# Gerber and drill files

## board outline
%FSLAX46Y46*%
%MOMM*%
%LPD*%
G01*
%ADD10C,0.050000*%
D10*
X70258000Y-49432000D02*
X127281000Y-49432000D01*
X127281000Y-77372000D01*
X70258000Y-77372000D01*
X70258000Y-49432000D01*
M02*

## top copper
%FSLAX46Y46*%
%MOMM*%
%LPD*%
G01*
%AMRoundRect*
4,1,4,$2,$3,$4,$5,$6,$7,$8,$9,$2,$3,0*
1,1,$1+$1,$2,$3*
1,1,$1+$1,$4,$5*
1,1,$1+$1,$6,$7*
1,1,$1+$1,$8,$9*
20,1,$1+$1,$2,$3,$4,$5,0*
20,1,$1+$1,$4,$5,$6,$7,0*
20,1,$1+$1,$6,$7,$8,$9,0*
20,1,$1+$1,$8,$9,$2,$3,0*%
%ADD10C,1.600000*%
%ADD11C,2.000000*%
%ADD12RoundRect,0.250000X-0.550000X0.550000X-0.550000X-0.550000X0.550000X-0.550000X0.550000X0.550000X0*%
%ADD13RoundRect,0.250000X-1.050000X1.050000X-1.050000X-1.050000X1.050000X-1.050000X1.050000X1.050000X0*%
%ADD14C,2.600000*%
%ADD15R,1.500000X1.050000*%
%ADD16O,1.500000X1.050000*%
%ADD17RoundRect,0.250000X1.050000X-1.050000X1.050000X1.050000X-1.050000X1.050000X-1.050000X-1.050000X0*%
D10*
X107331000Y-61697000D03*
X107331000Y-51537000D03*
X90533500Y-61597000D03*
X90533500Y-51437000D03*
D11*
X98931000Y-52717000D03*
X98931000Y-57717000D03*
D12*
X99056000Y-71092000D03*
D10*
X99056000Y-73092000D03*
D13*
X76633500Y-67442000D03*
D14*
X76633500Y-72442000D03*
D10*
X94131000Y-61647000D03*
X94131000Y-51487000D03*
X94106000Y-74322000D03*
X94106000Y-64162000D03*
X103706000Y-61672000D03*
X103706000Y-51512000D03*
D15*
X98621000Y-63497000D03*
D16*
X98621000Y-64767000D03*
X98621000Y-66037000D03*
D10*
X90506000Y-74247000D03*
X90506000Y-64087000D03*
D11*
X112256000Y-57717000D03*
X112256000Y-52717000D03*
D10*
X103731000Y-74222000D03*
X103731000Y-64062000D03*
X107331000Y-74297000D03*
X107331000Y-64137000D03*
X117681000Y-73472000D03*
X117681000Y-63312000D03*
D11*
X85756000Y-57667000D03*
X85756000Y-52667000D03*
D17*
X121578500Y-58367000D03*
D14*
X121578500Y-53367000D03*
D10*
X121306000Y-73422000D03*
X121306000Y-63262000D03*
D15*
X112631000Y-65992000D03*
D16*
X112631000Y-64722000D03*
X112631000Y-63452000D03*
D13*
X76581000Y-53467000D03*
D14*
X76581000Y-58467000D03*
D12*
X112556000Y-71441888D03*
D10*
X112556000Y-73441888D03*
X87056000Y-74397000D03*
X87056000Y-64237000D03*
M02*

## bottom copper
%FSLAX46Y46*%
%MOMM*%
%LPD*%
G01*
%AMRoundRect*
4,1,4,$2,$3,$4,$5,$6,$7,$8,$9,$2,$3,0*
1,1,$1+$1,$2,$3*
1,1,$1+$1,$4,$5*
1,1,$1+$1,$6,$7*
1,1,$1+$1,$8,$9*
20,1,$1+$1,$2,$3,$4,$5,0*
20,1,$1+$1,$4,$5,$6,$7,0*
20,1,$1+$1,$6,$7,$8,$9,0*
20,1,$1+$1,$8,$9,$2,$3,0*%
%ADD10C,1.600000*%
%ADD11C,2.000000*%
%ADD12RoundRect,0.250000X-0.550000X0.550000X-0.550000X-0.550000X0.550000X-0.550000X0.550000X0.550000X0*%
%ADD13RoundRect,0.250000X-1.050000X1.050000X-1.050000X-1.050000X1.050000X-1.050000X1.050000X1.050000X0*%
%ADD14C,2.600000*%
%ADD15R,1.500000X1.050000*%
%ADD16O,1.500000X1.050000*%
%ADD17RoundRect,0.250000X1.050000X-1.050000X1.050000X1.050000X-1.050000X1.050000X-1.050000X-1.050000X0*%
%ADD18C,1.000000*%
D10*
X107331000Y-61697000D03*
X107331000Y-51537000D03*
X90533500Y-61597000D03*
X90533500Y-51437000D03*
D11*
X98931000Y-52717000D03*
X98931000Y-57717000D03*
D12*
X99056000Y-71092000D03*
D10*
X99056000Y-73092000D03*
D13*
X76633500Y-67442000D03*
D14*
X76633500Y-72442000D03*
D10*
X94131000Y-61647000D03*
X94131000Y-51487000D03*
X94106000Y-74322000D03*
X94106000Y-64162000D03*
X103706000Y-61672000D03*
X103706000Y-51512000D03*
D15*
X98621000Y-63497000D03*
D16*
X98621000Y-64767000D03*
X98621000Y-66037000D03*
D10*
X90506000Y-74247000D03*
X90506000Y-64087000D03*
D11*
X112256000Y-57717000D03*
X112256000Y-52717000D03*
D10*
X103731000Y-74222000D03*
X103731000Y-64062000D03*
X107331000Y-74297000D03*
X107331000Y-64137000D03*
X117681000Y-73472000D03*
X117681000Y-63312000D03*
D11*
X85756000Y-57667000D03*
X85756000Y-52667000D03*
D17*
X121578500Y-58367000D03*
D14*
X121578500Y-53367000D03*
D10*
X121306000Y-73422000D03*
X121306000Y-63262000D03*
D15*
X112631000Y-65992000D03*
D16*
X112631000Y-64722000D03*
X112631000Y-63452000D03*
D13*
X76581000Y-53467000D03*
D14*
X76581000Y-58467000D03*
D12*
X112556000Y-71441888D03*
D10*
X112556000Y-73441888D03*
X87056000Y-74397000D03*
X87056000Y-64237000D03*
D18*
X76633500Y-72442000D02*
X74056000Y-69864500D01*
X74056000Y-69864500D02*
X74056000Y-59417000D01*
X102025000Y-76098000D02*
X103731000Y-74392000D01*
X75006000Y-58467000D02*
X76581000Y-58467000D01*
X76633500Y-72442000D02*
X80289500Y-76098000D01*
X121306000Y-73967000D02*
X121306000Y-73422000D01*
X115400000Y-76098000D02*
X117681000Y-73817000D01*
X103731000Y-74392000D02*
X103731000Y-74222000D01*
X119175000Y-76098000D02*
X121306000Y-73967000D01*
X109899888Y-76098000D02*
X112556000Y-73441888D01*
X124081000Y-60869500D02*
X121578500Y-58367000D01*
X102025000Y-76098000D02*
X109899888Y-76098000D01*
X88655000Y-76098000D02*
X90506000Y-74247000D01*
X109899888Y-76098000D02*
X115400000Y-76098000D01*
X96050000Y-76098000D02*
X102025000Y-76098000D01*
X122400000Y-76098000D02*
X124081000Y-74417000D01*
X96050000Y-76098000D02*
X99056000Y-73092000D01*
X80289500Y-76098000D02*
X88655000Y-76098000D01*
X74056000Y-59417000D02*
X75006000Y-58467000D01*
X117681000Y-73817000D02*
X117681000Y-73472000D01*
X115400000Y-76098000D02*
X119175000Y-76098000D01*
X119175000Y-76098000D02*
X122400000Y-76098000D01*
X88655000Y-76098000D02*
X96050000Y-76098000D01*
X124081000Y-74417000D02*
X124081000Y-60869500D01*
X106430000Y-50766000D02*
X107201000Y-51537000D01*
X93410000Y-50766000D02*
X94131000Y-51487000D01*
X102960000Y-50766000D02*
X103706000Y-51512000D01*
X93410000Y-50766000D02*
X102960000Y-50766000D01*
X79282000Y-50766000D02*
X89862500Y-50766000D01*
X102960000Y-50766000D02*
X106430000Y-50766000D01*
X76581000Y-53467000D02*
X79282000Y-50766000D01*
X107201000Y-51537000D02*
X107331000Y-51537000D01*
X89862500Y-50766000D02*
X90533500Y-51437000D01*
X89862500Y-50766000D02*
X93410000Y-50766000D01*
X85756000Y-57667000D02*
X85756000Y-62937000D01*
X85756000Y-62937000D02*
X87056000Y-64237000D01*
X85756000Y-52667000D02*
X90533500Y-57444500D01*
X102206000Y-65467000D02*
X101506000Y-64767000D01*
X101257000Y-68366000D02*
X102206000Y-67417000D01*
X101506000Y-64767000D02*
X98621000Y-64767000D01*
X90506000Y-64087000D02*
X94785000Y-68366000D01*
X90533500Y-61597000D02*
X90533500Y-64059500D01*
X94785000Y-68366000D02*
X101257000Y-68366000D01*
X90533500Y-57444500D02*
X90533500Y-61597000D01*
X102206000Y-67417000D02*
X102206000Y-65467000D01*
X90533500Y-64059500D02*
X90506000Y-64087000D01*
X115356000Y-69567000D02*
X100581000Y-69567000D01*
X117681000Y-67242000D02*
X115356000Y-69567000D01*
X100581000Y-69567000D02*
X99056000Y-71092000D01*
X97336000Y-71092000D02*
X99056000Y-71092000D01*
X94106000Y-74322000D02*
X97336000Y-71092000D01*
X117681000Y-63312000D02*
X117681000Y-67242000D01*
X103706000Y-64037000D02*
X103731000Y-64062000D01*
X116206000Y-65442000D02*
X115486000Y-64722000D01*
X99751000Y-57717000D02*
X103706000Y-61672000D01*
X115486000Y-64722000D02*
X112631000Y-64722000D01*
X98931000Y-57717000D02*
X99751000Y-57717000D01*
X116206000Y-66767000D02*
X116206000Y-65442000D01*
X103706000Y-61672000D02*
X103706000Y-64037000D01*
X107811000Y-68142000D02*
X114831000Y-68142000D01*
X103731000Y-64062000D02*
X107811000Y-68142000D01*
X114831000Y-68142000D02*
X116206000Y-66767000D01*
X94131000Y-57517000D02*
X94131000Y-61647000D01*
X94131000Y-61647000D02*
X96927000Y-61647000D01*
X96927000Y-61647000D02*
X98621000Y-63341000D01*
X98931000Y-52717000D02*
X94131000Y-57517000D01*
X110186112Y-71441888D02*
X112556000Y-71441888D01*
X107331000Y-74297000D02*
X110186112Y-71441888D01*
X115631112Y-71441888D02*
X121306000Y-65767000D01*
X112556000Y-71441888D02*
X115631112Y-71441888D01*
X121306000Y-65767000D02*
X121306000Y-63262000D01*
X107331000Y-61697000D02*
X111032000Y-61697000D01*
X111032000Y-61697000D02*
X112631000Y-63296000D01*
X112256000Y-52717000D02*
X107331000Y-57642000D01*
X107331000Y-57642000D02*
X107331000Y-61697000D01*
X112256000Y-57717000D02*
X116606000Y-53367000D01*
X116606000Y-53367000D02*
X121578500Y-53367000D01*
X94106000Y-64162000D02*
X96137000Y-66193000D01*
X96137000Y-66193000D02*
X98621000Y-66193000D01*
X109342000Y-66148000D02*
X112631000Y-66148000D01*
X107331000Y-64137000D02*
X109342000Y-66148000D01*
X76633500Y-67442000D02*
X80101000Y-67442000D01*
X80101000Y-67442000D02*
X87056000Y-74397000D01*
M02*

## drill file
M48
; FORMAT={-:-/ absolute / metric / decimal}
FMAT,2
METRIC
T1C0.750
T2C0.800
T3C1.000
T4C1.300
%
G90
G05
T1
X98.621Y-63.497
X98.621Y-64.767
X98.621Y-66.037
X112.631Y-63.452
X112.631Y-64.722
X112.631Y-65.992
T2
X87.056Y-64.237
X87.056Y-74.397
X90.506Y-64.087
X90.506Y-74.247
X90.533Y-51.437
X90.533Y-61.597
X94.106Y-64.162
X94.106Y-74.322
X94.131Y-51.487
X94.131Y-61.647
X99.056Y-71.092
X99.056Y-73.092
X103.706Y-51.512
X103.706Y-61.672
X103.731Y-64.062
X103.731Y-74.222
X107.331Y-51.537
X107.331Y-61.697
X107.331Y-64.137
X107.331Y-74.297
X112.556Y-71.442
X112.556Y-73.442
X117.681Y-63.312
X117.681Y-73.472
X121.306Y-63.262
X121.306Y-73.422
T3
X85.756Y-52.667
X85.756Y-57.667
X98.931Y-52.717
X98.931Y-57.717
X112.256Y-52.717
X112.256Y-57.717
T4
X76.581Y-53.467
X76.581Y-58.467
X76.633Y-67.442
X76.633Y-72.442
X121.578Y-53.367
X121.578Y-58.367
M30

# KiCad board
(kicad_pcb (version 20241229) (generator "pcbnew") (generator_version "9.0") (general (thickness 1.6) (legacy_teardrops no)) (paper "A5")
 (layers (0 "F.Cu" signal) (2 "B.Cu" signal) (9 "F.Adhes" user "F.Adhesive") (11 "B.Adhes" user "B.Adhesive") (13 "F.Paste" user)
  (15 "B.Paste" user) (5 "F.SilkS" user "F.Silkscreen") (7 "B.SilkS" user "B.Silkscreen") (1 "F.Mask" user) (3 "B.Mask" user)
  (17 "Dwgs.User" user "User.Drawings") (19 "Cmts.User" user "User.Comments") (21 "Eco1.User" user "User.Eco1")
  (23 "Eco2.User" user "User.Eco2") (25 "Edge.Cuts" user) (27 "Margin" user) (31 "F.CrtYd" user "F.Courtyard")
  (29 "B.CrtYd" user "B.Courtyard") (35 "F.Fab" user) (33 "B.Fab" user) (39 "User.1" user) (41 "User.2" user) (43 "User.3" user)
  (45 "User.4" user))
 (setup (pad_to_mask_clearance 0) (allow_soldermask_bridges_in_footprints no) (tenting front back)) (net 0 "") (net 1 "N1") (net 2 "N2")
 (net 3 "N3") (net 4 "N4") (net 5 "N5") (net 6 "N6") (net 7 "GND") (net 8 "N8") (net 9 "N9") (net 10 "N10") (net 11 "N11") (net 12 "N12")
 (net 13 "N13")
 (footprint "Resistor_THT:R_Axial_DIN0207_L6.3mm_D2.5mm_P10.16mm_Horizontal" (layer "F.Cu") (at 107.331 61.697 90)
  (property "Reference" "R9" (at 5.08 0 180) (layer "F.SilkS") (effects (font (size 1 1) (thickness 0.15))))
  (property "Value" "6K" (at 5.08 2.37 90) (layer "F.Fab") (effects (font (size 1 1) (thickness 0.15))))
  (pad "1" thru_hole circle (at 0 0 90) (size 1.6 1.6) (drill 0.8) (layers "*.Cu" "*.Mask") (remove_unused_layers no) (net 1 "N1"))
  (pad "2" thru_hole circle (at 10.16 0 90) (size 1.6 1.6) (drill 0.8) (layers "*.Cu" "*.Mask") (remove_unused_layers no) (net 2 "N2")))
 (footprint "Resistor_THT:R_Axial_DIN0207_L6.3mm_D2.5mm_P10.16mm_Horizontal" (layer "F.Cu") (at 90.5335 61.597 90)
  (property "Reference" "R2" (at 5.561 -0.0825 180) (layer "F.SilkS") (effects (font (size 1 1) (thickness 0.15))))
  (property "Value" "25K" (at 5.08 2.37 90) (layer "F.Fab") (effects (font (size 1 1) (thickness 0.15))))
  (pad "1" thru_hole circle (at 0 0 90) (size 1.6 1.6) (drill 0.8) (layers "*.Cu" "*.Mask") (remove_unused_layers no) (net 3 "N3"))
  (pad "2" thru_hole circle (at 10.16 0 90) (size 1.6 1.6) (drill 0.8) (layers "*.Cu" "*.Mask") (remove_unused_layers no) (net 2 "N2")))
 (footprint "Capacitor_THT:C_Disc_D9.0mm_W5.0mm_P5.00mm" (layer "F.Cu") (at 98.931 52.717 -90)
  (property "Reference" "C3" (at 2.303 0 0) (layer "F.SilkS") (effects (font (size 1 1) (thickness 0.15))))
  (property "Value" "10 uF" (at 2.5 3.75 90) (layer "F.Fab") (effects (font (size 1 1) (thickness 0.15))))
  (pad "1" thru_hole circle (at 0 0 270) (size 2 2) (drill 1) (layers "*.Cu" "*.Mask") (remove_unused_layers no) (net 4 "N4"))
  (pad "2" thru_hole circle (at 5 0 270) (size 2 2) (drill 1) (layers "*.Cu" "*.Mask") (remove_unused_layers no) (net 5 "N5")))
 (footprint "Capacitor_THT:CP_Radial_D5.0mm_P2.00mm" (layer "F.Cu") (at 99.056 71.092 -90)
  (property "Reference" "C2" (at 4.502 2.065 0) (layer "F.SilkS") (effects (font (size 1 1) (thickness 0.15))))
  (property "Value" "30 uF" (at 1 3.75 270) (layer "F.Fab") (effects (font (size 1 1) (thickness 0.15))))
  (pad "1" thru_hole roundrect (at 0 0 270) (size 1.6 1.6) (drill 0.8) (layers "*.Cu" "*.Mask") (remove_unused_layers no)
   (roundrect_rratio 0.15625) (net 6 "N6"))
  (pad "2" thru_hole circle (at 2 0 270) (size 1.6 1.6) (drill 0.8) (layers "*.Cu" "*.Mask") (remove_unused_layers no) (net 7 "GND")))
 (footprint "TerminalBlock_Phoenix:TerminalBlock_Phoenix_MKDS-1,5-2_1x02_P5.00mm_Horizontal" (layer "F.Cu") (at 76.6335 67.442 -90)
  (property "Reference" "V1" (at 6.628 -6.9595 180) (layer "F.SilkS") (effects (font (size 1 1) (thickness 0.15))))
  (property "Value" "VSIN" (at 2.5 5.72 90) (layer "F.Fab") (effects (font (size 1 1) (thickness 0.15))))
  (pad "1" thru_hole roundrect (at 0 0 270) (size 2.6 2.6) (drill 1.3) (layers "*.Cu" "*.Mask") (remove_unused_layers no)
   (roundrect_rratio 0.096154) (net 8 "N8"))
  (pad "2" thru_hole circle (at 5 0 270) (size 2.6 2.6) (drill 1.3) (layers "*.Cu" "*.Mask") (remove_unused_layers no) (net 7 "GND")))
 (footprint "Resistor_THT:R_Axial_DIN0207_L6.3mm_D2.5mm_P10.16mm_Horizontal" (layer "F.Cu") (at 94.131 61.647 90)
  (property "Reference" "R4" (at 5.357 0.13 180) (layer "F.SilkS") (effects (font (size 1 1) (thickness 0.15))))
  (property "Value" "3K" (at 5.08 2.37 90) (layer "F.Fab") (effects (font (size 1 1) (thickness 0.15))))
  (pad "1" thru_hole circle (at 0 0 90) (size 1.6 1.6) (drill 0.8) (layers "*.Cu" "*.Mask") (remove_unused_layers no) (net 4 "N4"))
  (pad "2" thru_hole circle (at 10.16 0 90) (size 1.6 1.6) (drill 0.8) (layers "*.Cu" "*.Mask") (remove_unused_layers no) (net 2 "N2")))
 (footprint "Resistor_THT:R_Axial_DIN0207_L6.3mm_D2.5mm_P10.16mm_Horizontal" (layer "F.Cu") (at 94.106 74.322 90)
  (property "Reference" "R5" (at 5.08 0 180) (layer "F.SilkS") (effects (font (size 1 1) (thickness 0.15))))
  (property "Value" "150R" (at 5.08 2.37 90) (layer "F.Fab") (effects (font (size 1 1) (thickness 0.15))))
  (pad "1" thru_hole circle (at 0 0 90) (size 1.6 1.6) (drill 0.8) (layers "*.Cu" "*.Mask") (remove_unused_layers no) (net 6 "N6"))
  (pad "2" thru_hole circle (at 10.16 0 90) (size 1.6 1.6) (drill 0.8) (layers "*.Cu" "*.Mask") (remove_unused_layers no) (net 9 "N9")))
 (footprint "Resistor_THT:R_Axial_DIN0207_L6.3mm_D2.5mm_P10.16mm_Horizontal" (layer "F.Cu") (at 103.706 61.672 90)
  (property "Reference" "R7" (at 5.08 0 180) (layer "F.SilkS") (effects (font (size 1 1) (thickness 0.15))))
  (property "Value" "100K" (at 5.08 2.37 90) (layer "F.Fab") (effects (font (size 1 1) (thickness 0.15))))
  (pad "1" thru_hole circle (at 0 0 90) (size 1.6 1.6) (drill 0.8) (layers "*.Cu" "*.Mask") (remove_unused_layers no) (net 5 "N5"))
  (pad "2" thru_hole circle (at 10.16 0 90) (size 1.6 1.6) (drill 0.8) (layers "*.Cu" "*.Mask") (remove_unused_layers no) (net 2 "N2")))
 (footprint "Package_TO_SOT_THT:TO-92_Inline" (layer "F.Cu") (at 98.621 63.497 -90)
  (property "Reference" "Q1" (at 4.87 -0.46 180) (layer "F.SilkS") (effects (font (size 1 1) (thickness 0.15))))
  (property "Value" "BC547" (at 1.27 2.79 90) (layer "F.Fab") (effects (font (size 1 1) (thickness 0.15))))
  (pad "1" thru_hole rect (at 0 0 270) (size 1.05 1.5) (drill 0.75) (layers "*.Cu" "*.Mask") (remove_unused_layers no) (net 4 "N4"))
  (pad "2" thru_hole oval (at 1.27 0 270) (size 1.05 1.5) (drill 0.75) (layers "*.Cu" "*.Mask") (remove_unused_layers no) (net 3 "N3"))
  (pad "3" thru_hole oval (at 2.54 0 270) (size 1.05 1.5) (drill 0.75) (layers "*.Cu" "*.Mask") (remove_unused_layers no) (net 9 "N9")))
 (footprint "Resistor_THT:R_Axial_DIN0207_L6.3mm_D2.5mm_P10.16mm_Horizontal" (layer "F.Cu") (at 90.506 74.247 90)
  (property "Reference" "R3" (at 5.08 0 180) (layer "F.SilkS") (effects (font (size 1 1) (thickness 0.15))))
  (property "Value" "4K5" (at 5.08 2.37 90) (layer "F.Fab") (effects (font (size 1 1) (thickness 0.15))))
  (pad "1" thru_hole circle (at 0 0 90) (size 1.6 1.6) (drill 0.8) (layers "*.Cu" "*.Mask") (remove_unused_layers no) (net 7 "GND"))
  (pad "2" thru_hole circle (at 10.16 0 90) (size 1.6 1.6) (drill 0.8) (layers "*.Cu" "*.Mask") (remove_unused_layers no) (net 3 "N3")))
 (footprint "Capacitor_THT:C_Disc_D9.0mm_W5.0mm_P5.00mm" (layer "F.Cu") (at 112.256 57.717 90)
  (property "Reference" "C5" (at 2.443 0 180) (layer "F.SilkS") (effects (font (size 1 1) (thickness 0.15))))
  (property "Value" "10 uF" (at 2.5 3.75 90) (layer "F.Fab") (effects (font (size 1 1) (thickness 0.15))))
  (pad "1" thru_hole circle (at 0 0 90) (size 2 2) (drill 1) (layers "*.Cu" "*.Mask") (remove_unused_layers no) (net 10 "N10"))
  (pad "2" thru_hole circle (at 5 0 90) (size 2 2) (drill 1) (layers "*.Cu" "*.Mask") (remove_unused_layers no) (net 1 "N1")))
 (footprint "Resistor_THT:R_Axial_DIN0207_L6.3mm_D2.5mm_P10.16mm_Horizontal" (layer "F.Cu") (at 103.731 74.222 90)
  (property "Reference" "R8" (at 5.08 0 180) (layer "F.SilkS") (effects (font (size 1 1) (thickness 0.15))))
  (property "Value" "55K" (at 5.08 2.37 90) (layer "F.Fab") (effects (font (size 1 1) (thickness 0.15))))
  (pad "1" thru_hole circle (at 0 0 90) (size 1.6 1.6) (drill 0.8) (layers "*.Cu" "*.Mask") (remove_unused_layers no) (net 7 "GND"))
  (pad "2" thru_hole circle (at 10.16 0 90) (size 1.6 1.6) (drill 0.8) (layers "*.Cu" "*.Mask") (remove_unused_layers no) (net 5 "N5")))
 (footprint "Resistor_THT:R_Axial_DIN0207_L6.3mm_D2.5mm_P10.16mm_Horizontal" (layer "F.Cu") (at 107.331 74.297 90)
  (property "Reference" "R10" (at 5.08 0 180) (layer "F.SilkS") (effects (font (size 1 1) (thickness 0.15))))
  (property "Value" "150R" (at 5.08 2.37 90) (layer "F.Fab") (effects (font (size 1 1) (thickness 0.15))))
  (pad "1" thru_hole circle (at 0 0 90) (size 1.6 1.6) (drill 0.8) (layers "*.Cu" "*.Mask") (remove_unused_layers no) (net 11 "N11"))
  (pad "2" thru_hole circle (at 10.16 0 90) (size 1.6 1.6) (drill 0.8) (layers "*.Cu" "*.Mask") (remove_unused_layers no) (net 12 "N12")))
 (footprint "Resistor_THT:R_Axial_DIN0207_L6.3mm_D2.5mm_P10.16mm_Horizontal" (layer "F.Cu") (at 117.681 73.472 90)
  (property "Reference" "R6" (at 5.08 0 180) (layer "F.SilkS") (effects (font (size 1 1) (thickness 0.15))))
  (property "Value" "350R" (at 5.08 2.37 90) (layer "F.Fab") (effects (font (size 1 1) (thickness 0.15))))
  (pad "1" thru_hole circle (at 0 0 90) (size 1.6 1.6) (drill 0.8) (layers "*.Cu" "*.Mask") (remove_unused_layers no) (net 7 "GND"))
  (pad "2" thru_hole circle (at 10.16 0 90) (size 1.6 1.6) (drill 0.8) (layers "*.Cu" "*.Mask") (remove_unused_layers no) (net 6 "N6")))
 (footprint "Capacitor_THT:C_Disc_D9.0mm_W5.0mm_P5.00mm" (layer "F.Cu") (at 85.756 57.667 90)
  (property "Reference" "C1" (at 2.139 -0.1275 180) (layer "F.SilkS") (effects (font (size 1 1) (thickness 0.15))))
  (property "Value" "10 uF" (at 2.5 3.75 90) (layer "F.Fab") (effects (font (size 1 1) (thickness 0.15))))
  (pad "1" thru_hole circle (at 0 0 90) (size 2 2) (drill 1) (layers "*.Cu" "*.Mask") (remove_unused_layers no) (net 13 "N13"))
  (pad "2" thru_hole circle (at 5 0 90) (size 2 2) (drill 1) (layers "*.Cu" "*.Mask") (remove_unused_layers no) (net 3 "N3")))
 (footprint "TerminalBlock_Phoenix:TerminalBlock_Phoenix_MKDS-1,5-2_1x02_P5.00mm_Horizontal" (layer "F.Cu") (at 121.5785 58.367 90)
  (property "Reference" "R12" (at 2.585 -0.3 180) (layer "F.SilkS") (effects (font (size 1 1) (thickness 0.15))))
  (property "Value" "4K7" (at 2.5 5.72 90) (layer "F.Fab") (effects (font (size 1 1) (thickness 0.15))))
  (pad "1" thru_hole roundrect (at 0 0 90) (size 2.6 2.6) (drill 1.3) (layers "*.Cu" "*.Mask") (remove_unused_layers no)
   (roundrect_rratio 0.096154) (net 7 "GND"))
  (pad "2" thru_hole circle (at 5 0 90) (size 2.6 2.6) (drill 1.3) (layers "*.Cu" "*.Mask") (remove_unused_layers no) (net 10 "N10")))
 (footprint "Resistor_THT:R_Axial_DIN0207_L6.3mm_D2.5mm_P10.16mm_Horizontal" (layer "F.Cu") (at 121.306 73.422 90)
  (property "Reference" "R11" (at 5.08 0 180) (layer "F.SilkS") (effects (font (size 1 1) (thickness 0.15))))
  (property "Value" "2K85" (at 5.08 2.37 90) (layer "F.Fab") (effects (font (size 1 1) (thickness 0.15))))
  (pad "1" thru_hole circle (at 0 0 90) (size 1.6 1.6) (drill 0.8) (layers "*.Cu" "*.Mask") (remove_unused_layers no) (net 7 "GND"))
  (pad "2" thru_hole circle (at 10.16 0 90) (size 1.6 1.6) (drill 0.8) (layers "*.Cu" "*.Mask") (remove_unused_layers no) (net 11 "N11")))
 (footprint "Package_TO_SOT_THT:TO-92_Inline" (layer "F.Cu") (at 112.631 65.992 90)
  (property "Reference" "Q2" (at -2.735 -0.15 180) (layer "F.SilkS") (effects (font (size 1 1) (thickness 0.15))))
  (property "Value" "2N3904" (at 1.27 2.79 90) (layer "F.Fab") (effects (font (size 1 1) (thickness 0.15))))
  (pad "1" thru_hole rect (at 0 0 90) (size 1.05 1.5) (drill 0.75) (layers "*.Cu" "*.Mask") (remove_unused_layers no) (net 12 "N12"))
  (pad "2" thru_hole oval (at 1.27 0 90) (size 1.05 1.5) (drill 0.75) (layers "*.Cu" "*.Mask") (remove_unused_layers no) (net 5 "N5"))
  (pad "3" thru_hole oval (at 2.54 0 90) (size 1.05 1.5) (drill 0.75) (layers "*.Cu" "*.Mask") (remove_unused_layers no) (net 1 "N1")))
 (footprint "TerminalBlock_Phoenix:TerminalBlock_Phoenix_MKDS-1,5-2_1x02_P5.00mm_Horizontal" (layer "F.Cu") (at 76.581 53.467 -90)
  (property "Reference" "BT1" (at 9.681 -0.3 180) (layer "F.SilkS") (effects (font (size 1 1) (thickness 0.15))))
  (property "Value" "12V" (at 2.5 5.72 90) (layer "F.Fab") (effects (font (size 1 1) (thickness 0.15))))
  (pad "1" thru_hole roundrect (at 0 0 270) (size 2.6 2.6) (drill 1.3) (layers "*.Cu" "*.Mask") (remove_unused_layers no)
   (roundrect_rratio 0.096154) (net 2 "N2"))
  (pad "2" thru_hole circle (at 5 0 270) (size 2.6 2.6) (drill 1.3) (layers "*.Cu" "*.Mask") (remove_unused_layers no) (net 7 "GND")))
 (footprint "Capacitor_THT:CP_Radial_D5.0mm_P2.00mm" (layer "F.Cu") (at 112.556 71.441888 -90)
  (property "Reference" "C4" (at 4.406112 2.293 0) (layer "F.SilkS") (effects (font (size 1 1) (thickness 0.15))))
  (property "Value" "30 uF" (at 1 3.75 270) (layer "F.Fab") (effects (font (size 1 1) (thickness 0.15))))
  (pad "1" thru_hole roundrect (at 0 0 270) (size 1.6 1.6) (drill 0.8) (layers "*.Cu" "*.Mask") (remove_unused_layers no)
   (roundrect_rratio 0.15625) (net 11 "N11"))
  (pad "2" thru_hole circle (at 2 0 270) (size 1.6 1.6) (drill 0.8) (layers "*.Cu" "*.Mask") (remove_unused_layers no) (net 7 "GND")))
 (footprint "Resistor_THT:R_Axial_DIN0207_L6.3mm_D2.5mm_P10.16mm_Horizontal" (layer "F.Cu") (at 87.056 74.397 90)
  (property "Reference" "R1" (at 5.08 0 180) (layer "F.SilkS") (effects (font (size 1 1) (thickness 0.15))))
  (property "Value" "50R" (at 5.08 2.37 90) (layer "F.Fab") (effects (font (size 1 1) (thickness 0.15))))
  (pad "1" thru_hole circle (at 0 0 90) (size 1.6 1.6) (drill 0.8) (layers "*.Cu" "*.Mask") (remove_unused_layers no) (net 8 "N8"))
  (pad "2" thru_hole circle (at 10.16 0 90) (size 1.6 1.6) (drill 0.8) (layers "*.Cu" "*.Mask") (remove_unused_layers no) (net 13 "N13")))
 (gr_rect (start 70.258 49.432) (end 127.281 77.372) (stroke (width 0.05) (type default)) (fill no) (layer "Edge.Cuts"))
 (segment (start 76.6335 72.442) (end 74.056 69.8645) (width 1) (layer "B.Cu") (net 7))
 (segment (start 74.056 69.8645) (end 74.056 59.417) (width 1) (layer "B.Cu") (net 7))
 (segment (start 102.025 76.098) (end 103.731 74.392) (width 1) (layer "B.Cu") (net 7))
 (segment (start 75.006 58.467) (end 76.581 58.467) (width 1) (layer "B.Cu") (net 7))
 (segment (start 76.6335 72.442) (end 80.2895 76.098) (width 1) (layer "B.Cu") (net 7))
 (segment (start 121.306 73.967) (end 121.306 73.422) (width 1) (layer "B.Cu") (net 7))
 (segment (start 115.4 76.098) (end 117.681 73.817) (width 1) (layer "B.Cu") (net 7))
 (segment (start 103.731 74.392) (end 103.731 74.222) (width 1) (layer "B.Cu") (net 7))
 (segment (start 119.175 76.098) (end 121.306 73.967) (width 1) (layer "B.Cu") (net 7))
 (segment (start 109.899888 76.098) (end 112.556 73.441888) (width 1) (layer "B.Cu") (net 7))
 (segment (start 124.081 60.8695) (end 121.5785 58.367) (width 1) (layer "B.Cu") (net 7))
 (segment (start 102.025 76.098) (end 109.899888 76.098) (width 1) (layer "B.Cu") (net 7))
 (segment (start 88.655 76.098) (end 90.506 74.247) (width 1) (layer "B.Cu") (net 7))
 (segment (start 109.899888 76.098) (end 115.4 76.098) (width 1) (layer "B.Cu") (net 7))
 (segment (start 96.05 76.098) (end 102.025 76.098) (width 1) (layer "B.Cu") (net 7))
 (segment (start 122.4 76.098) (end 124.081 74.417) (width 1) (layer "B.Cu") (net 7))
 (segment (start 96.05 76.098) (end 99.056 73.092) (width 1) (layer "B.Cu") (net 7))
 (segment (start 80.2895 76.098) (end 88.655 76.098) (width 1) (layer "B.Cu") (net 7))
 (segment (start 74.056 59.417) (end 75.006 58.467) (width 1) (layer "B.Cu") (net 7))
 (segment (start 117.681 73.817) (end 117.681 73.472) (width 1) (layer "B.Cu") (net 7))
 (segment (start 115.4 76.098) (end 119.175 76.098) (width 1) (layer "B.Cu") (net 7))
 (segment (start 119.175 76.098) (end 122.4 76.098) (width 1) (layer "B.Cu") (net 7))
 (segment (start 88.655 76.098) (end 96.05 76.098) (width 1) (layer "B.Cu") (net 7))
 (segment (start 124.081 74.417) (end 124.081 60.8695) (width 1) (layer "B.Cu") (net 7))
 (segment (start 106.43 50.766) (end 107.201 51.537) (width 1) (layer "B.Cu") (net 2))
 (segment (start 93.41 50.766) (end 94.131 51.487) (width 1) (layer "B.Cu") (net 2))
 (segment (start 102.96 50.766) (end 103.706 51.512) (width 1) (layer "B.Cu") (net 2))
 (segment (start 93.41 50.766) (end 102.96 50.766) (width 1) (layer "B.Cu") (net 2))
 (segment (start 79.282 50.766) (end 89.8625 50.766) (width 1) (layer "B.Cu") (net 2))
 (segment (start 102.96 50.766) (end 106.43 50.766) (width 1) (layer "B.Cu") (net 2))
 (segment (start 76.581 53.467) (end 79.282 50.766) (width 1) (layer "B.Cu") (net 2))
 (segment (start 107.201 51.537) (end 107.331 51.537) (width 1) (layer "B.Cu") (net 2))
 (segment (start 89.8625 50.766) (end 90.5335 51.437) (width 1) (layer "B.Cu") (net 2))
 (segment (start 89.8625 50.766) (end 93.41 50.766) (width 1) (layer "B.Cu") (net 2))
 (segment (start 85.756 57.667) (end 85.756 62.937) (width 1) (layer "B.Cu") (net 13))
 (segment (start 85.756 62.937) (end 87.056 64.237) (width 1) (layer "B.Cu") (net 13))
 (segment (start 85.756 52.667) (end 90.5335 57.4445) (width 1) (layer "B.Cu") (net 3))
 (segment (start 102.206 65.467) (end 101.506 64.767) (width 1) (layer "B.Cu") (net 3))
 (segment (start 101.257 68.366) (end 102.206 67.417) (width 1) (layer "B.Cu") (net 3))
 (segment (start 101.506 64.767) (end 98.621 64.767) (width 1) (layer "B.Cu") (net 3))
 (segment (start 90.506 64.087) (end 94.785 68.366) (width 1) (layer "B.Cu") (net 3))
 (segment (start 90.5335 61.597) (end 90.5335 64.0595) (width 1) (layer "B.Cu") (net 3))
 (segment (start 94.785 68.366) (end 101.257 68.366) (width 1) (layer "B.Cu") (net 3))
 (segment (start 90.5335 57.4445) (end 90.5335 61.597) (width 1) (layer "B.Cu") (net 3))
 (segment (start 102.206 67.417) (end 102.206 65.467) (width 1) (layer "B.Cu") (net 3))
 (segment (start 90.5335 64.0595) (end 90.506 64.087) (width 1) (layer "B.Cu") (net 3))
 (segment (start 115.356 69.567) (end 100.581 69.567) (width 1) (layer "B.Cu") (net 6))
 (segment (start 117.681 67.242) (end 115.356 69.567) (width 1) (layer "B.Cu") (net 6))
 (segment (start 100.581 69.567) (end 99.056 71.092) (width 1) (layer "B.Cu") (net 6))
 (segment (start 97.336 71.092) (end 99.056 71.092) (width 1) (layer "B.Cu") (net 6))
 (segment (start 94.106 74.322) (end 97.336 71.092) (width 1) (layer "B.Cu") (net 6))
 (segment (start 117.681 63.312) (end 117.681 67.242) (width 1) (layer "B.Cu") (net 6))
 (segment (start 103.706 64.037) (end 103.731 64.062) (width 1) (layer "B.Cu") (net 5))
 (segment (start 116.206 65.442) (end 115.486 64.722) (width 1) (layer "B.Cu") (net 5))
 (segment (start 99.751 57.717) (end 103.706 61.672) (width 1) (layer "B.Cu") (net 5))
 (segment (start 115.486 64.722) (end 112.631 64.722) (width 1) (layer "B.Cu") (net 5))
 (segment (start 98.931 57.717) (end 99.751 57.717) (width 1) (layer "B.Cu") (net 5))
 (segment (start 116.206 66.767) (end 116.206 65.442) (width 1) (layer "B.Cu") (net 5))
 (segment (start 103.706 61.672) (end 103.706 64.037) (width 1) (layer "B.Cu") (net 5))
 (segment (start 107.811 68.142) (end 114.831 68.142) (width 1) (layer "B.Cu") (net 5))
 (segment (start 103.731 64.062) (end 107.811 68.142) (width 1) (layer "B.Cu") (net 5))
 (segment (start 114.831 68.142) (end 116.206 66.767) (width 1) (layer "B.Cu") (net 5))
 (segment (start 94.131 57.517) (end 94.131 61.647) (width 1) (layer "B.Cu") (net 4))
 (segment (start 94.131 61.647) (end 96.927 61.647) (width 1) (layer "B.Cu") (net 4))
 (segment (start 96.927 61.647) (end 98.621 63.341) (width 1) (layer "B.Cu") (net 4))
 (segment (start 98.931 52.717) (end 94.131 57.517) (width 1) (layer "B.Cu") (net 4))
 (segment (start 110.186112 71.441888) (end 112.556 71.441888) (width 1) (layer "B.Cu") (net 11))
 (segment (start 107.331 74.297) (end 110.186112 71.441888) (width 1) (layer "B.Cu") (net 11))
 (segment (start 115.631112 71.441888) (end 121.306 65.767) (width 1) (layer "B.Cu") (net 11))
 (segment (start 112.556 71.441888) (end 115.631112 71.441888) (width 1) (layer "B.Cu") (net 11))
 (segment (start 121.306 65.767) (end 121.306 63.262) (width 1) (layer "B.Cu") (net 11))
 (segment (start 107.331 61.697) (end 111.032 61.697) (width 1) (layer "B.Cu") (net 1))
 (segment (start 111.032 61.697) (end 112.631 63.296) (width 1) (layer "B.Cu") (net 1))
 (segment (start 112.256 52.717) (end 107.331 57.642) (width 1) (layer "B.Cu") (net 1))
 (segment (start 107.331 57.642) (end 107.331 61.697) (width 1) (layer "B.Cu") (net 1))
 (segment (start 112.256 57.717) (end 116.606 53.367) (width 1) (layer "B.Cu") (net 10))
 (segment (start 116.606 53.367) (end 121.5785 53.367) (width 1) (layer "B.Cu") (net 10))
 (segment (start 94.106 64.162) (end 96.137 66.193) (width 1) (layer "B.Cu") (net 9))
 (segment (start 96.137 66.193) (end 98.621 66.193) (width 1) (layer "B.Cu") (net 9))
 (segment (start 109.342 66.148) (end 112.631 66.148) (width 1) (layer "B.Cu") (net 12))
 (segment (start 107.331 64.137) (end 109.342 66.148) (width 1) (layer "B.Cu") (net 12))
 (segment (start 76.6335 67.442) (end 80.101 67.442) (width 1) (layer "B.Cu") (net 8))
 (segment (start 80.101 67.442) (end 87.056 74.397) (width 1) (layer "B.Cu") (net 8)))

